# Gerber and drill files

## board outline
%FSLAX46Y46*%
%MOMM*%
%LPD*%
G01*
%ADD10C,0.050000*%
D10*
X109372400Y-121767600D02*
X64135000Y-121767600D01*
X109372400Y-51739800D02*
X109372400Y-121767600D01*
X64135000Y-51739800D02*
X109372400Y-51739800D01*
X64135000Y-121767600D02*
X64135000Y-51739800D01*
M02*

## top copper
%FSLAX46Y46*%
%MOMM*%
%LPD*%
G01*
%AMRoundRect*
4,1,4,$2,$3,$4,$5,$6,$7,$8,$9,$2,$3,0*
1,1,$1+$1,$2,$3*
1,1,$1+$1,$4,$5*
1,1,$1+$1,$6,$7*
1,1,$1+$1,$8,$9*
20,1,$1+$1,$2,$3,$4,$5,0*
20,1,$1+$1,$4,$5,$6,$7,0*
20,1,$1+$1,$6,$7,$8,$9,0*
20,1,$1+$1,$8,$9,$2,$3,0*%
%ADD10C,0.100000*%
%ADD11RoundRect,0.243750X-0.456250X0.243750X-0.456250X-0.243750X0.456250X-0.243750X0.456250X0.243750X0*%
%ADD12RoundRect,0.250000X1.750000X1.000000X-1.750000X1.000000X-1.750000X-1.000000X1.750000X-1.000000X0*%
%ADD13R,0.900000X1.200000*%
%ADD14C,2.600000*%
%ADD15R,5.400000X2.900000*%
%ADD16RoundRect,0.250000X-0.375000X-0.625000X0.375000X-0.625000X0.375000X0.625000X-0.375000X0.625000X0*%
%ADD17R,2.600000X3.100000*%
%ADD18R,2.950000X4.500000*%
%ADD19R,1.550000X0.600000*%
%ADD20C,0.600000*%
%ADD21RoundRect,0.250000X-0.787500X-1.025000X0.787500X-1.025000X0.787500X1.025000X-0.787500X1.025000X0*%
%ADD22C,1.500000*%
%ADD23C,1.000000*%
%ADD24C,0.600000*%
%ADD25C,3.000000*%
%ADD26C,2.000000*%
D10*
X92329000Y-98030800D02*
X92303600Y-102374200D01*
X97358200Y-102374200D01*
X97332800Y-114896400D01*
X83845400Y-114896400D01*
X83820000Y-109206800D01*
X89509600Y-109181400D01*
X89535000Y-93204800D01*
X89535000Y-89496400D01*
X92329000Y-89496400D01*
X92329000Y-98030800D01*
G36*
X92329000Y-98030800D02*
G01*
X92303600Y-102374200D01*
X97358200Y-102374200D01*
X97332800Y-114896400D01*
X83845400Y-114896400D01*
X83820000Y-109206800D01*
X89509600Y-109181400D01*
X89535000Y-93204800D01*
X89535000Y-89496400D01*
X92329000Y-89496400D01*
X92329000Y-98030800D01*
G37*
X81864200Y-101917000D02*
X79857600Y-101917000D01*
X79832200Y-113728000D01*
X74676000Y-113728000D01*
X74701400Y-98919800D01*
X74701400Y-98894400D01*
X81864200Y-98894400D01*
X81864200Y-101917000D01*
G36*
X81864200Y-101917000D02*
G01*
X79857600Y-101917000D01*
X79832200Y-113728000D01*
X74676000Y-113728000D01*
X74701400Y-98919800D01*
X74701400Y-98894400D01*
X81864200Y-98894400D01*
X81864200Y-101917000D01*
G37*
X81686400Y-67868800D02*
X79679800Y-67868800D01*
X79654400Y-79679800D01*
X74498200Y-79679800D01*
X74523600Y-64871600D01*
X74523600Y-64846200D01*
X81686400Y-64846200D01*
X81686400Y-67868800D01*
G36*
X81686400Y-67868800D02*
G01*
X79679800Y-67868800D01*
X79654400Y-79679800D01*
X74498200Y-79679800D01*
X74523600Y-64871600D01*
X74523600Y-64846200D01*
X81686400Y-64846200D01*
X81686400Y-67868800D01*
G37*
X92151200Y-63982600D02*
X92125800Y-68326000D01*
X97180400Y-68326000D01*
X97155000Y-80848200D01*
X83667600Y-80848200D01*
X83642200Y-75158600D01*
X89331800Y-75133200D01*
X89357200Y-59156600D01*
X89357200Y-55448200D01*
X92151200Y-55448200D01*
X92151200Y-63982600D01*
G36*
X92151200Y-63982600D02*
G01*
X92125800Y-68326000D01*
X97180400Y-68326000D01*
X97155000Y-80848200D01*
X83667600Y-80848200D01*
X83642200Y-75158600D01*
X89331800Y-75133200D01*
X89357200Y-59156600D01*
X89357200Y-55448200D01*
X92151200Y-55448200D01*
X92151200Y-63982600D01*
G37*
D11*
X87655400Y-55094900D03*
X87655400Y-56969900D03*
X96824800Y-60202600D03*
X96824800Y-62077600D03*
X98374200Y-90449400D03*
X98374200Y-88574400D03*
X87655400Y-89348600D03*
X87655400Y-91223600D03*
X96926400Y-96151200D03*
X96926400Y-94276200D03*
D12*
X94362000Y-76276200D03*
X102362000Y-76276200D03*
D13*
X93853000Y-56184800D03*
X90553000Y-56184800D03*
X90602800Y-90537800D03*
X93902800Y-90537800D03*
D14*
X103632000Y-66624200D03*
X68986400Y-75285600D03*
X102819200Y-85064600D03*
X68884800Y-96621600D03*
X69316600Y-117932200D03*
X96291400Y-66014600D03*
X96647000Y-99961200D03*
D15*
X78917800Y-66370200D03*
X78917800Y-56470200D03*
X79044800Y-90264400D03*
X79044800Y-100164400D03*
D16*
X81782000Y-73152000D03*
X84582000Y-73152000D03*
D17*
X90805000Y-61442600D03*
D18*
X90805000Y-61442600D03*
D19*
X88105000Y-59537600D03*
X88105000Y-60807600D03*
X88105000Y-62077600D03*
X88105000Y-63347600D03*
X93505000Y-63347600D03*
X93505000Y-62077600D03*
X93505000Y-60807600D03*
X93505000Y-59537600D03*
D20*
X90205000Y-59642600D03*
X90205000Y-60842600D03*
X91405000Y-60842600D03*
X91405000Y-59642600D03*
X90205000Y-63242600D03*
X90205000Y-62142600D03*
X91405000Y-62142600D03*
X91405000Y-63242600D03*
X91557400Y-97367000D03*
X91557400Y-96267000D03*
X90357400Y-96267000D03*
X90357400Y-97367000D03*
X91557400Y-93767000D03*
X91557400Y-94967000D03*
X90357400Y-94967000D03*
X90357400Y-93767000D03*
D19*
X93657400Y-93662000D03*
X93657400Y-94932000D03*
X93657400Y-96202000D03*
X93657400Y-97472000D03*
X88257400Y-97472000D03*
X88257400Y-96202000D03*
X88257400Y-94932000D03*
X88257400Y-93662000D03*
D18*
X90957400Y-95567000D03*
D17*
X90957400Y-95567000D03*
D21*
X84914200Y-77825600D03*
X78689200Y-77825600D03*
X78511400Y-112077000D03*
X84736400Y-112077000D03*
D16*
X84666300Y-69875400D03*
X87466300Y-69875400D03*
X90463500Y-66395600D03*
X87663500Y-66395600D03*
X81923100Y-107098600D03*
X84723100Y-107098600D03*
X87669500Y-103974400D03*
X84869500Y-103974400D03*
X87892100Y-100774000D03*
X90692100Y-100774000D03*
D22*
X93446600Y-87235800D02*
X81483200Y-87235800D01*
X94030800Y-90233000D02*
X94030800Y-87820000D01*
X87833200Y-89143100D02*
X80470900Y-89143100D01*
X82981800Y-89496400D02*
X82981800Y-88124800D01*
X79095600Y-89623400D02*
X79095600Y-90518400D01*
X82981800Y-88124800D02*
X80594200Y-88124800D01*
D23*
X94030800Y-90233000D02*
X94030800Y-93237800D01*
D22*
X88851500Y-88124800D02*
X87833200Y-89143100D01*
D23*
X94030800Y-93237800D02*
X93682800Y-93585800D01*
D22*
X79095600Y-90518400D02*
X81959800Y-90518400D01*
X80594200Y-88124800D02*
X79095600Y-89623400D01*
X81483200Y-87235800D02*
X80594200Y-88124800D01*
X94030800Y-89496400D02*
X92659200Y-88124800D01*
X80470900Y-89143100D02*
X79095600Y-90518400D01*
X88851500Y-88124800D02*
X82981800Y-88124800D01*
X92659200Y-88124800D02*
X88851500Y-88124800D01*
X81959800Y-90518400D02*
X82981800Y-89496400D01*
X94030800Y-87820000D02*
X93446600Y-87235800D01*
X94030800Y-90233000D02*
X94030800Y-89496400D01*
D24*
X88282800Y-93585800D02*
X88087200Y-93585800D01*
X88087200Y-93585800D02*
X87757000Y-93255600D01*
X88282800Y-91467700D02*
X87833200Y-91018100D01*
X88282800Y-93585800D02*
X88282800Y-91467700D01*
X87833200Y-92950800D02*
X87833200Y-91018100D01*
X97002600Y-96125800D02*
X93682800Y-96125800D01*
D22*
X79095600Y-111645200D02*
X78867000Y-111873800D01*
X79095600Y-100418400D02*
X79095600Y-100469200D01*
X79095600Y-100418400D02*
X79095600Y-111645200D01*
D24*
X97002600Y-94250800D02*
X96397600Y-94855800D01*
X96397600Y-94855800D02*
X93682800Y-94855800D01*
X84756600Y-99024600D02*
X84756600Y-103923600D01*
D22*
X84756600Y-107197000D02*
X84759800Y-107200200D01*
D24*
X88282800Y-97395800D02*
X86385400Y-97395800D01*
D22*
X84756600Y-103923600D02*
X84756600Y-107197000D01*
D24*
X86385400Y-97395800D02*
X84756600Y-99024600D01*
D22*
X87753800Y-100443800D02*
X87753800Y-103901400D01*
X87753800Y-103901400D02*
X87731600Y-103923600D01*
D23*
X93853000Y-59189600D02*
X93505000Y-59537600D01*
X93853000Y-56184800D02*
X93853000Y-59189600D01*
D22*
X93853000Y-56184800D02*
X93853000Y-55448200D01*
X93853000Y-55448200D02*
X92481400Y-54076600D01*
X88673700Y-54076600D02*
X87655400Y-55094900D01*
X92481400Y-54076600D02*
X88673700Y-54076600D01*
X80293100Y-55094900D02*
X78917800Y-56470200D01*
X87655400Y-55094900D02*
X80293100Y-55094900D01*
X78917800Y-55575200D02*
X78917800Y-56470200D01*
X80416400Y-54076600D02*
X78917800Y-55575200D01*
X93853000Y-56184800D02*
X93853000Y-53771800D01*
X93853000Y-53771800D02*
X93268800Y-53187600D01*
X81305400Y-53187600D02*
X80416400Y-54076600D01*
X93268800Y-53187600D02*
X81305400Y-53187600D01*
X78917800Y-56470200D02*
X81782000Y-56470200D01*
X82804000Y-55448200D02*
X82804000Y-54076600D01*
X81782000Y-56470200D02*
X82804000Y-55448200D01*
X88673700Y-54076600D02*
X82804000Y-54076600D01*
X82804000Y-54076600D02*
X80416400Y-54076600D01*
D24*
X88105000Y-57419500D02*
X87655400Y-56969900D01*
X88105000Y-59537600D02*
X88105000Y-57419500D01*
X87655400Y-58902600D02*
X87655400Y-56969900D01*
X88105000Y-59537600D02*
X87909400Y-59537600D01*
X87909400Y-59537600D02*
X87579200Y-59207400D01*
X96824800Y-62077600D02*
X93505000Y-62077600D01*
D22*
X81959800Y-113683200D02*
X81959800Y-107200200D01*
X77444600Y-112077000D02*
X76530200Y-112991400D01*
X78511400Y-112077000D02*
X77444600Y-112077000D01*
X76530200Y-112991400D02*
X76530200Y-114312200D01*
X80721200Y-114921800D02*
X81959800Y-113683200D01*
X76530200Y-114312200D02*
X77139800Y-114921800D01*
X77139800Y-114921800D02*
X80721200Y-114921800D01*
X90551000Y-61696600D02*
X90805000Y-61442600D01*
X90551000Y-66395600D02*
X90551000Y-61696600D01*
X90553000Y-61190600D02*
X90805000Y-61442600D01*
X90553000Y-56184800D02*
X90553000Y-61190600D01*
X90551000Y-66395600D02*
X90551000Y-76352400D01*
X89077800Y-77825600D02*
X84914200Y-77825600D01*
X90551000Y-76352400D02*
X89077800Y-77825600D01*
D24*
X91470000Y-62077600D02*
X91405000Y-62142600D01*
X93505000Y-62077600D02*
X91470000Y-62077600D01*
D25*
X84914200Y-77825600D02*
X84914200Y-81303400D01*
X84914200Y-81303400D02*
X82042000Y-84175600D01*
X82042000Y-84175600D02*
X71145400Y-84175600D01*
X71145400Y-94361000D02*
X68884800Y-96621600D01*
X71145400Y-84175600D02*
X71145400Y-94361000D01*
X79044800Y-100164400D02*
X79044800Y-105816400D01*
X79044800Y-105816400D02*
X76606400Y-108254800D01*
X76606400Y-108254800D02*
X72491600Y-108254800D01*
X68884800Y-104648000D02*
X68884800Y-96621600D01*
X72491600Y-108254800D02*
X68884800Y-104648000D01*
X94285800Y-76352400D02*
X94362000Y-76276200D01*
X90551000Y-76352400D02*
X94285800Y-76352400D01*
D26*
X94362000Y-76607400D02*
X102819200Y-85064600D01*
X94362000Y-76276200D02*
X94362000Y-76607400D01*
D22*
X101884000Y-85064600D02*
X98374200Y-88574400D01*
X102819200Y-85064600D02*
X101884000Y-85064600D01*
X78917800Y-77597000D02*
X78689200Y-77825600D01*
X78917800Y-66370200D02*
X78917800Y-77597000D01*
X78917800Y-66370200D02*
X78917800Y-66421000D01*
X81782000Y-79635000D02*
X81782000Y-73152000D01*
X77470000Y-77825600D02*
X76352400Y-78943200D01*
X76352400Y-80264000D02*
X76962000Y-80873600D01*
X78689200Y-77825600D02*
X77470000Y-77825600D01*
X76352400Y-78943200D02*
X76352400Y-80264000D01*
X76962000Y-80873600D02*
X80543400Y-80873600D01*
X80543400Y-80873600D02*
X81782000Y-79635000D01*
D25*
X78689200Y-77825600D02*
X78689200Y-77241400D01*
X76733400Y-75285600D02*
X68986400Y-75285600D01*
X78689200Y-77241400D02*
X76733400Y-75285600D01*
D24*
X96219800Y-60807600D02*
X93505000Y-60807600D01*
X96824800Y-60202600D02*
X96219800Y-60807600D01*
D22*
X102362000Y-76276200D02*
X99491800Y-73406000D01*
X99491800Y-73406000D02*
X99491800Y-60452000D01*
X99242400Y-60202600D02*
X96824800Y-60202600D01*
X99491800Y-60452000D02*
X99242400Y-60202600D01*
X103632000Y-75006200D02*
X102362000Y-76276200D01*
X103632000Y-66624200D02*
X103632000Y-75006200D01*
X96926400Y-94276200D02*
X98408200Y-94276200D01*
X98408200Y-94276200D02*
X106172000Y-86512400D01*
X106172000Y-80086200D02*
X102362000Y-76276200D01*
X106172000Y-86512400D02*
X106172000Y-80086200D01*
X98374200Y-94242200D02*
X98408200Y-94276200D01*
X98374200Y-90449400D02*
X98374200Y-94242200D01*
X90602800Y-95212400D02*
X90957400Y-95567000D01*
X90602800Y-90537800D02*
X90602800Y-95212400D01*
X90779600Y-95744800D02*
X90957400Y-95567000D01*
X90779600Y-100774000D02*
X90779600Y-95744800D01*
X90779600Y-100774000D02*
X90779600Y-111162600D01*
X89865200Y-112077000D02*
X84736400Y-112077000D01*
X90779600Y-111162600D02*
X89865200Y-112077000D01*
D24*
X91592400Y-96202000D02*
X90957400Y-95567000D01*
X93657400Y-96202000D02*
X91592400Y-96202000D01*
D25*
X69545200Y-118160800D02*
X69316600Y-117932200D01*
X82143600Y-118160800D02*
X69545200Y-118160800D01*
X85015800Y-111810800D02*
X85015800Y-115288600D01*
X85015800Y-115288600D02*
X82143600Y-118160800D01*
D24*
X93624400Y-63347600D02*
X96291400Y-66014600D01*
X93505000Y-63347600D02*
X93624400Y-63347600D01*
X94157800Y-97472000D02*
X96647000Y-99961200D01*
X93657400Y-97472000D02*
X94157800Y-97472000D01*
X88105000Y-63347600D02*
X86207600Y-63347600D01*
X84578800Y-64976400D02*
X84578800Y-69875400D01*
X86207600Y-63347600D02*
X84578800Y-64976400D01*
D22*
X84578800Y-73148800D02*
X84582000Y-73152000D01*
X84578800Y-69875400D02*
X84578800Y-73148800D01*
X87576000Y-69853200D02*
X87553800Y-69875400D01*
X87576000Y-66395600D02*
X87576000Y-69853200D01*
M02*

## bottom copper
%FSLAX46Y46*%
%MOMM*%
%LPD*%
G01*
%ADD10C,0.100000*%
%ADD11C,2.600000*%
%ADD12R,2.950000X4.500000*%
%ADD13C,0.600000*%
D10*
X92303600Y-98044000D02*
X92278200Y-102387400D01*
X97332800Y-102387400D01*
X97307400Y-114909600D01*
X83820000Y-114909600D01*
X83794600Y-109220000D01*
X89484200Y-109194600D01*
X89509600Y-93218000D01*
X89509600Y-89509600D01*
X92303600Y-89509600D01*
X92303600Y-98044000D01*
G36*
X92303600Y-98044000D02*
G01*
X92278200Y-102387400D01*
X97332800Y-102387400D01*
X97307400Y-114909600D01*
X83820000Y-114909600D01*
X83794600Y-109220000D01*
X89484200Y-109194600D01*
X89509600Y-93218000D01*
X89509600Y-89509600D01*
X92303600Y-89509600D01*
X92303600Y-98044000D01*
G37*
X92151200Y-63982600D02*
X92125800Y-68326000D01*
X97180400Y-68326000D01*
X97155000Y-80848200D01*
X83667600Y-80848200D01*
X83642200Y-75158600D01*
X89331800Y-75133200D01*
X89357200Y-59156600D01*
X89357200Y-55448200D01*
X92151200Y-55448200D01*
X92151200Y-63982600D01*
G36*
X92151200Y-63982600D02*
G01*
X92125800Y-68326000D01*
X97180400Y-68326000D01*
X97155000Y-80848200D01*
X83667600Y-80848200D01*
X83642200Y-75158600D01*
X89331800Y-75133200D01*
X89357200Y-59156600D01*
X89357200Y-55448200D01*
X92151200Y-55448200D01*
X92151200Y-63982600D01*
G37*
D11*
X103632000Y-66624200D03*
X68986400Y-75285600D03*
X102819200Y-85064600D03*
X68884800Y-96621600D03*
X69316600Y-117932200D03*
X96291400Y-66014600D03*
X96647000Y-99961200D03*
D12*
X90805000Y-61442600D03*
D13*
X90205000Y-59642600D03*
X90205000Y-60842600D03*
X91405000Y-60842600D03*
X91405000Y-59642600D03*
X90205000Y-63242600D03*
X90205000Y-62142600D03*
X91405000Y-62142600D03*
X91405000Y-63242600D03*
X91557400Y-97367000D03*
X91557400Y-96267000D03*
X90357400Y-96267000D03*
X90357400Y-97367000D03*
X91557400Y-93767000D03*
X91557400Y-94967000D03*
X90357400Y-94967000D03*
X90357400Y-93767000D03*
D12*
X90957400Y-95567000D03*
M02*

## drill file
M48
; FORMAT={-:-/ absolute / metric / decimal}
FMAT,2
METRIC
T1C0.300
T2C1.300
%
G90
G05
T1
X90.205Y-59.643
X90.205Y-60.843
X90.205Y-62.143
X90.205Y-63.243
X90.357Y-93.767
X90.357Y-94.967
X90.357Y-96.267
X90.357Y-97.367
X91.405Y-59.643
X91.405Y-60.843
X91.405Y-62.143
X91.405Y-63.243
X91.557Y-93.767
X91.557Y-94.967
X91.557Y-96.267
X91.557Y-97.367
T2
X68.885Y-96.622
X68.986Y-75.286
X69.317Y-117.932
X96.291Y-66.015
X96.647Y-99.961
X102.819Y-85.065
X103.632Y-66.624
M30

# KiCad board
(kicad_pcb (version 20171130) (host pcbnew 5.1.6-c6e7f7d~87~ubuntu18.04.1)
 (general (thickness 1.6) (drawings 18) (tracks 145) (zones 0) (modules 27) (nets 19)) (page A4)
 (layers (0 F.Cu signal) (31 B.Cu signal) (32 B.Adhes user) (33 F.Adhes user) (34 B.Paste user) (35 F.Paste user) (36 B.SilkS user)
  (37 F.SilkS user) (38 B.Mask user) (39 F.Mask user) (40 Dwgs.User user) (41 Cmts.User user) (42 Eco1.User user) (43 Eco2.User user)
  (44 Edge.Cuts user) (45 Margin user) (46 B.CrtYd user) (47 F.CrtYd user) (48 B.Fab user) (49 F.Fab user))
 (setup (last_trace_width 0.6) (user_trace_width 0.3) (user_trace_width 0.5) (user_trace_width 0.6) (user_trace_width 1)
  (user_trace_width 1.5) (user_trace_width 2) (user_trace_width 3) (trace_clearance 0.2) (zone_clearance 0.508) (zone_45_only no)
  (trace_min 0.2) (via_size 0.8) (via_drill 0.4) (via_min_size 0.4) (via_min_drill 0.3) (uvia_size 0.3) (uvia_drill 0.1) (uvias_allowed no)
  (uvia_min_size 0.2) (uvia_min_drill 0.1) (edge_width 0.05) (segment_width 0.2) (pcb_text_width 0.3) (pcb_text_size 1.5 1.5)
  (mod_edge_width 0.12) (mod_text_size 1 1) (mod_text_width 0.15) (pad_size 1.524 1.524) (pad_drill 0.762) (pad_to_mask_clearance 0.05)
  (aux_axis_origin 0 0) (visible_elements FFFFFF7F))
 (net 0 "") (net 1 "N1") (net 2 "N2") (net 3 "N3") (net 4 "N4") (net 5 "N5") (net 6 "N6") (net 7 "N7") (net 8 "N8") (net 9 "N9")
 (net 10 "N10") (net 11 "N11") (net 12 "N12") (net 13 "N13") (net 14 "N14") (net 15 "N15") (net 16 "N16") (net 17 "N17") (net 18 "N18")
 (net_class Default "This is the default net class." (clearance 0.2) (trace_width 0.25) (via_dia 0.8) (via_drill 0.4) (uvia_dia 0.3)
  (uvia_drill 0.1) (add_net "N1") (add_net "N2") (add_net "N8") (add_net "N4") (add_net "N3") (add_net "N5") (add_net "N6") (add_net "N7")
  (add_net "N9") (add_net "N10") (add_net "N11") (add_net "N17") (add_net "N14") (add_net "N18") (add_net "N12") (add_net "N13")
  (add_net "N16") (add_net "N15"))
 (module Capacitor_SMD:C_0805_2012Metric (layer F.Cu) (at 87.6554 56.0324 270)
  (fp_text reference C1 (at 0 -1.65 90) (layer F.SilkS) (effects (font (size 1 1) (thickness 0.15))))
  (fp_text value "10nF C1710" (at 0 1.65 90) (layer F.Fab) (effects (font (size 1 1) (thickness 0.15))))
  (pad 1 smd roundrect (at -0.9375 0 270) (size 0.975 1.4) (layers F.Cu F.Paste F.Mask) (roundrect_rratio 0.25) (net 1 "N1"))
  (pad 2 smd roundrect (at 0.9375 0 270) (size 0.975 1.4) (layers F.Cu F.Paste F.Mask) (roundrect_rratio 0.25) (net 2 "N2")))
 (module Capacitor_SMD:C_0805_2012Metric (layer F.Cu) (at 96.8248 61.1401 270)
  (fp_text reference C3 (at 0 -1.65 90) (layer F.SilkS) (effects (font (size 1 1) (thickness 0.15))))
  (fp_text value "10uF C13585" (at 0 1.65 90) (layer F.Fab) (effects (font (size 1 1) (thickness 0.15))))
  (pad 1 smd roundrect (at -0.9375 0 270) (size 0.975 1.4) (layers F.Cu F.Paste F.Mask) (roundrect_rratio 0.25) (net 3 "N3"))
  (pad 2 smd roundrect (at 0.9375 0 270) (size 0.975 1.4) (layers F.Cu F.Paste F.Mask) (roundrect_rratio 0.25) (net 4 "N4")))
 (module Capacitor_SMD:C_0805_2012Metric (layer F.Cu) (at 98.3742 89.5119 270)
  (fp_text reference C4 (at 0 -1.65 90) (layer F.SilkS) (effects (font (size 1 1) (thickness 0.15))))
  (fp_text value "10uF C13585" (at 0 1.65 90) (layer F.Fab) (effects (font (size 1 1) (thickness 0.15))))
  (pad 2 smd roundrect (at 0.9375 0 270) (size 0.975 1.4) (layers F.Cu F.Paste F.Mask) (roundrect_rratio 0.25) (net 3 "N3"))
  (pad 1 smd roundrect (at -0.9375 0 270) (size 0.975 1.4) (layers F.Cu F.Paste F.Mask) (roundrect_rratio 0.25) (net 4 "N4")))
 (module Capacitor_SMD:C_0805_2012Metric (layer F.Cu) (at 87.6554 90.2861 270)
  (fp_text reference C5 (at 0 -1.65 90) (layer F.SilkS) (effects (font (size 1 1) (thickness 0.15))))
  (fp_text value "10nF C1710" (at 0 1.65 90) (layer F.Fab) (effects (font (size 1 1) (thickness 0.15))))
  (pad 1 smd roundrect (at -0.9375 0 270) (size 0.975 1.4) (layers F.Cu F.Paste F.Mask) (roundrect_rratio 0.25) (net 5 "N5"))
  (pad 2 smd roundrect (at 0.9375 0 270) (size 0.975 1.4) (layers F.Cu F.Paste F.Mask) (roundrect_rratio 0.25) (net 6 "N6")))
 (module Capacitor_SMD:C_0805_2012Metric (layer F.Cu) (at 96.9264 95.2137 270)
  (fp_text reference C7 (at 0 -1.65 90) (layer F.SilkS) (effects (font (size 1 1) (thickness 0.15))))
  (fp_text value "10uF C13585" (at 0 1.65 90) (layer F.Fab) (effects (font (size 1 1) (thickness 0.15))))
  (pad 2 smd roundrect (at 0.9375 0 270) (size 0.975 1.4) (layers F.Cu F.Paste F.Mask) (roundrect_rratio 0.25) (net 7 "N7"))
  (pad 1 smd roundrect (at -0.9375 0 270) (size 0.975 1.4) (layers F.Cu F.Paste F.Mask) (roundrect_rratio 0.25) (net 3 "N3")))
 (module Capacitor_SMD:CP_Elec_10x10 (layer F.Cu) (at 98.362 76.2762 180)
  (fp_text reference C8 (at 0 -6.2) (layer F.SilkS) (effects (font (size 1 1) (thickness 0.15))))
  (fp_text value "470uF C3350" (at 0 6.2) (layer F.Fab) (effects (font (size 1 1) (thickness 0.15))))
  (pad 2 smd roundrect (at 4 0 180) (size 4 2.5) (layers F.Cu F.Paste F.Mask) (roundrect_rratio 0.1) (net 4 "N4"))
  (pad 1 smd roundrect (at -4 0 180) (size 4 2.5) (layers F.Cu F.Paste F.Mask) (roundrect_rratio 0.1) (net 3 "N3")))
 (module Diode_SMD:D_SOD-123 (layer F.Cu) (at 92.203 56.1848 180)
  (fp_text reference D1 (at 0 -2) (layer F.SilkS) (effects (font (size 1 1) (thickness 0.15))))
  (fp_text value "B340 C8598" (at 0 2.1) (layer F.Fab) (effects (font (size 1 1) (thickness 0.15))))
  (pad 1 smd rect (at -1.65 0 180) (size 0.9 1.2) (layers F.Cu F.Paste F.Mask) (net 1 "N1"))
  (pad 2 smd rect (at 1.65 0 180) (size 0.9 1.2) (layers F.Cu F.Paste F.Mask) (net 4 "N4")))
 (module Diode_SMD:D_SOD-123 (layer F.Cu) (at 92.2528 90.5378 180)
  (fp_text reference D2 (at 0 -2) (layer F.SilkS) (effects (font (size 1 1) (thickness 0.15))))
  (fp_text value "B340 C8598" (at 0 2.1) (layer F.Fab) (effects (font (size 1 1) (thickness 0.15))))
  (pad 2 smd rect (at 1.65 0 180) (size 0.9 1.2) (layers F.Cu F.Paste F.Mask) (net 7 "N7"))
  (pad 1 smd rect (at -1.65 0 180) (size 0.9 1.2) (layers F.Cu F.Paste F.Mask) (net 5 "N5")))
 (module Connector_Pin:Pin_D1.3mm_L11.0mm (layer F.Cu) (at 103.632 66.6242)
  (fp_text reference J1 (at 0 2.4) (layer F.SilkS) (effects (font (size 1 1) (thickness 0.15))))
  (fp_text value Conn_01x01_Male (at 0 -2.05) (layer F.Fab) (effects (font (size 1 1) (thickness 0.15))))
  (pad 1 thru_hole circle (at 0 0) (size 2.6 2.6) (drill 1.3) (layers *.Cu *.Mask) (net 3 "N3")))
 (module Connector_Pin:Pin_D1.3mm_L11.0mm (layer F.Cu) (at 68.9864 75.2856)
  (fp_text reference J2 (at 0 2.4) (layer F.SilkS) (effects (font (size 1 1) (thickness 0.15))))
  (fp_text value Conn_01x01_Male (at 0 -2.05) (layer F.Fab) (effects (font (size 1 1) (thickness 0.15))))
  (pad 1 thru_hole circle (at 0 0) (size 2.6 2.6) (drill 1.3) (layers *.Cu *.Mask) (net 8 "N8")))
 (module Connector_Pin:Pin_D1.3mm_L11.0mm (layer F.Cu) (at 102.8192 85.0646)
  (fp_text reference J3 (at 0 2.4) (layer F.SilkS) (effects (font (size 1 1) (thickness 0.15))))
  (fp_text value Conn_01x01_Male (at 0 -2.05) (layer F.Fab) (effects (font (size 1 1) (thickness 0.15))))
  (pad 1 thru_hole circle (at 0 0) (size 2.6 2.6) (drill 1.3) (layers *.Cu *.Mask) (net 4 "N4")))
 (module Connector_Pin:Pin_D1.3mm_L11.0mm (layer F.Cu) (at 68.8848 96.6216)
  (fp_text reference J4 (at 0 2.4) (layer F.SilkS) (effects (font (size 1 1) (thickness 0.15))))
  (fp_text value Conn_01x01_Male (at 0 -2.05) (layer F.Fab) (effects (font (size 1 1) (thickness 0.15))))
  (pad 1 thru_hole circle (at 0 0) (size 2.6 2.6) (drill 1.3) (layers *.Cu *.Mask) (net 4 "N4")))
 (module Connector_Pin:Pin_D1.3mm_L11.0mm (layer F.Cu) (at 69.3166 117.9322)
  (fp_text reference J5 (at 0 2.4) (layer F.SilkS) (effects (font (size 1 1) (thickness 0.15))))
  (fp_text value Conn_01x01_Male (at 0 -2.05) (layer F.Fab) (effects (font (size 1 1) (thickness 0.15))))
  (pad 1 thru_hole circle (at 0 0) (size 2.6 2.6) (drill 1.3) (layers *.Cu *.Mask) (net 7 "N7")))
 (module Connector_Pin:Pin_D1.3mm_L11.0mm (layer F.Cu) (at 96.2914 66.0146)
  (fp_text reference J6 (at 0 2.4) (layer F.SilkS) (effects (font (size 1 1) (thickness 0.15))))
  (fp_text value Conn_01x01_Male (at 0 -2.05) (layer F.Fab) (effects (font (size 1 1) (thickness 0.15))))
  (pad 1 thru_hole circle (at 0 0) (size 2.6 2.6) (drill 1.3) (layers *.Cu *.Mask) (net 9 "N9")))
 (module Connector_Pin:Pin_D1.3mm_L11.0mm (layer F.Cu) (at 96.647 99.9612)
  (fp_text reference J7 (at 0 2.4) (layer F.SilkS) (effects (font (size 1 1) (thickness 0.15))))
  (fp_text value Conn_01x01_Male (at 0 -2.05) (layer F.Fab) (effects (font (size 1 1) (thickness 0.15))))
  (pad 1 thru_hole circle (at 0 0) (size 2.6 2.6) (drill 1.3) (layers *.Cu *.Mask) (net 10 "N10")))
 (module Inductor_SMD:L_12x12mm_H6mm (layer F.Cu) (at 78.9178 61.4202 90)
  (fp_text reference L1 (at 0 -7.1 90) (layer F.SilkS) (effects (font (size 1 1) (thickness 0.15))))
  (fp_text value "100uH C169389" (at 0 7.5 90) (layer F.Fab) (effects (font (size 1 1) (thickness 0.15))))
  (pad 1 smd rect (at -4.95 0 90) (size 2.9 5.4) (layers F.Cu F.Paste F.Mask) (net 8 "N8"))
  (pad 2 smd rect (at 4.95 0 90) (size 2.9 5.4) (layers F.Cu F.Paste F.Mask) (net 1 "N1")))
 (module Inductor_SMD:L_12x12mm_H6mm (layer F.Cu) (at 79.0448 95.2144 90)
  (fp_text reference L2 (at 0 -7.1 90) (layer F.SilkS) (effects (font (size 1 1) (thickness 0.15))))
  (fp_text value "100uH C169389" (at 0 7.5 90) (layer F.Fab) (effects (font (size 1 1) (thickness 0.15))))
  (pad 2 smd rect (at 4.95 0 90) (size 2.9 5.4) (layers F.Cu F.Paste F.Mask) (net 5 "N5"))
  (pad 1 smd rect (at -4.95 0 90) (size 2.9 5.4) (layers F.Cu F.Paste F.Mask) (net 4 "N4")))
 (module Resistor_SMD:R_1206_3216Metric (layer F.Cu) (at 83.182 73.152)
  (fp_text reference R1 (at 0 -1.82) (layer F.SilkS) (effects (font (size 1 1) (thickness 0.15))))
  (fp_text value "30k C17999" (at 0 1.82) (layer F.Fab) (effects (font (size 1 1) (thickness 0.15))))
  (pad 1 smd roundrect (at -1.4 0) (size 1.25 1.75) (layers F.Cu F.Paste F.Mask) (roundrect_rratio 0.2) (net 8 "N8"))
  (pad 2 smd roundrect (at 1.4 0) (size 1.25 1.75) (layers F.Cu F.Paste F.Mask) (roundrect_rratio 0.2) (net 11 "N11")))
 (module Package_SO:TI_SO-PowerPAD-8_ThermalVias (layer F.Cu) (at 90.805 61.4426)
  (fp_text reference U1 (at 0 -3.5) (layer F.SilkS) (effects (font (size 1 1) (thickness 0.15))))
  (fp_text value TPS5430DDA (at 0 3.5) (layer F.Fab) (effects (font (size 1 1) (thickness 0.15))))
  (pad 9 smd rect (at 0 0) (size 2.6 3.1) (layers F.Cu F.Paste F.Mask) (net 4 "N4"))
  (pad 9 smd rect (at 0 0) (size 2.95 4.5) (layers F.Cu) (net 4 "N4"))
  (pad 1 smd rect (at -2.7 -1.905) (size 1.55 0.6) (layers F.Cu F.Paste F.Mask) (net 2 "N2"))
  (pad 2 smd rect (at -2.7 -0.635) (size 1.55 0.6) (layers F.Cu F.Paste F.Mask) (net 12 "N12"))
  (pad 3 smd rect (at -2.7 0.635) (size 1.55 0.6) (layers F.Cu F.Paste F.Mask) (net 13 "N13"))
  (pad 4 smd rect (at -2.7 1.905) (size 1.55 0.6) (layers F.Cu F.Paste F.Mask) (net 11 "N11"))
  (pad 5 smd rect (at 2.7 1.905) (size 1.55 0.6) (layers F.Cu F.Paste F.Mask) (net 9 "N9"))
  (pad 6 smd rect (at 2.7 0.635) (size 1.55 0.6) (layers F.Cu F.Paste F.Mask) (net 4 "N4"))
  (pad 7 smd rect (at 2.7 -0.635) (size 1.55 0.6) (layers F.Cu F.Paste F.Mask) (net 3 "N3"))
  (pad 8 smd rect (at 2.7 -1.905) (size 1.55 0.6) (layers F.Cu F.Paste F.Mask) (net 1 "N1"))
  (pad 9 smd rect (at 0 0) (size 2.95 4.5) (layers B.Cu) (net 4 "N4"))
  (pad 9 thru_hole circle (at -0.6 -1.8) (size 0.6 0.6) (drill 0.3) (layers *.Cu) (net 4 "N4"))
  (pad 9 thru_hole circle (at -0.6 -0.6) (size 0.6 0.6) (drill 0.3) (layers *.Cu) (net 4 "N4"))
  (pad 9 thru_hole circle (at 0.6 -0.6) (size 0.6 0.6) (drill 0.3) (layers *.Cu) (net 4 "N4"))
  (pad 9 thru_hole circle (at 0.6 -1.8) (size 0.6 0.6) (drill 0.3) (layers *.Cu) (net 4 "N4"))
  (pad 9 thru_hole circle (at -0.6 1.8) (size 0.6 0.6) (drill 0.3) (layers *.Cu) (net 4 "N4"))
  (pad 9 thru_hole circle (at -0.6 0.7) (size 0.6 0.6) (drill 0.3) (layers *.Cu) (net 4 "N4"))
  (pad 9 thru_hole circle (at 0.6 0.7) (size 0.6 0.6) (drill 0.3) (layers *.Cu) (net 4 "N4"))
  (pad 9 thru_hole circle (at 0.6 1.8) (size 0.6 0.6) (drill 0.3) (layers *.Cu) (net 4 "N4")))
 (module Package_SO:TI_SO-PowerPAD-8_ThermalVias (layer F.Cu) (at 90.9574 95.567)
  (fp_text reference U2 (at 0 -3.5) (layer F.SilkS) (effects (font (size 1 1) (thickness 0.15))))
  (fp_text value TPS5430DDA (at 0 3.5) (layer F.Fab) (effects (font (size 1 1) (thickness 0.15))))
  (pad 9 thru_hole circle (at 0.6 1.8) (size 0.6 0.6) (drill 0.3) (layers *.Cu) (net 7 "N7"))
  (pad 9 thru_hole circle (at 0.6 0.7) (size 0.6 0.6) (drill 0.3) (layers *.Cu) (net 7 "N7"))
  (pad 9 thru_hole circle (at -0.6 0.7) (size 0.6 0.6) (drill 0.3) (layers *.Cu) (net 7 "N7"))
  (pad 9 thru_hole circle (at -0.6 1.8) (size 0.6 0.6) (drill 0.3) (layers *.Cu) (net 7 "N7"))
  (pad 9 thru_hole circle (at 0.6 -1.8) (size 0.6 0.6) (drill 0.3) (layers *.Cu) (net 7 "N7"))
  (pad 9 thru_hole circle (at 0.6 -0.6) (size 0.6 0.6) (drill 0.3) (layers *.Cu) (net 7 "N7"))
  (pad 9 thru_hole circle (at -0.6 -0.6) (size 0.6 0.6) (drill 0.3) (layers *.Cu) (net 7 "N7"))
  (pad 9 thru_hole circle (at -0.6 -1.8) (size 0.6 0.6) (drill 0.3) (layers *.Cu) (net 7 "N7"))
  (pad 9 smd rect (at 0 0) (size 2.95 4.5) (layers B.Cu) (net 7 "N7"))
  (pad 8 smd rect (at 2.7 -1.905) (size 1.55 0.6) (layers F.Cu F.Paste F.Mask) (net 5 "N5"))
  (pad 7 smd rect (at 2.7 -0.635) (size 1.55 0.6) (layers F.Cu F.Paste F.Mask) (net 3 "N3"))
  (pad 6 smd rect (at 2.7 0.635) (size 1.55 0.6) (layers F.Cu F.Paste F.Mask) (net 7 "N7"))
  (pad 5 smd rect (at 2.7 1.905) (size 1.55 0.6) (layers F.Cu F.Paste F.Mask) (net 10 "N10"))
  (pad 4 smd rect (at -2.7 1.905) (size 1.55 0.6) (layers F.Cu F.Paste F.Mask) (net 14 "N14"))
  (pad 3 smd rect (at -2.7 0.635) (size 1.55 0.6) (layers F.Cu F.Paste F.Mask) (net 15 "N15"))
  (pad 2 smd rect (at -2.7 -0.635) (size 1.55 0.6) (layers F.Cu F.Paste F.Mask) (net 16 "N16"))
  (pad 1 smd rect (at -2.7 -1.905) (size 1.55 0.6) (layers F.Cu F.Paste F.Mask) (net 6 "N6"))
  (pad 9 smd rect (at 0 0) (size 2.95 4.5) (layers F.Cu) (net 7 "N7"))
  (pad 9 smd rect (at 0 0) (size 2.6 3.1) (layers F.Cu F.Paste F.Mask) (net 7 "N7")))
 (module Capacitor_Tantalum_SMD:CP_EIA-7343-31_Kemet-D (layer F.Cu) (at 81.8017 77.8256)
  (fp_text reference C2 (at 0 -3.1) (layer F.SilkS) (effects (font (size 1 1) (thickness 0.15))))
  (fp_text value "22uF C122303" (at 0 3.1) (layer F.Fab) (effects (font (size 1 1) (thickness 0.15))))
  (pad 2 smd roundrect (at 3.1125 0) (size 2.075 2.55) (layers F.Cu F.Paste F.Mask) (roundrect_rratio 0.120482) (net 4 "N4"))
  (pad 1 smd roundrect (at -3.1125 0) (size 2.075 2.55) (layers F.Cu F.Paste F.Mask) (roundrect_rratio 0.120482) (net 8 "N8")))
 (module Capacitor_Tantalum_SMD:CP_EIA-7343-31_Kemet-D (layer F.Cu) (at 81.6239 112.077)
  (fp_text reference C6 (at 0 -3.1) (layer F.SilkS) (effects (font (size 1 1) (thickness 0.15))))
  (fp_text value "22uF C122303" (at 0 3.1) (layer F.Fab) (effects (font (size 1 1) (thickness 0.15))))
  (pad 1 smd roundrect (at -3.1125 0) (size 2.075 2.55) (layers F.Cu F.Paste F.Mask) (roundrect_rratio 0.120482) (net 4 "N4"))
  (pad 2 smd roundrect (at 3.1125 0) (size 2.075 2.55) (layers F.Cu F.Paste F.Mask) (roundrect_rratio 0.120482) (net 7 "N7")))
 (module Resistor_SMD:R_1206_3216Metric (layer F.Cu) (at 86.0663 69.8754)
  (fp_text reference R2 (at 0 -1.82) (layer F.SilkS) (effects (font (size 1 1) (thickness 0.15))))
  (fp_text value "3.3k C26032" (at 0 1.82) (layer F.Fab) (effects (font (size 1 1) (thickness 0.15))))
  (pad 1 smd roundrect (at -1.4 0) (size 1.25 1.75) (layers F.Cu F.Paste F.Mask) (roundrect_rratio 0.2) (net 11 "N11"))
  (pad 2 smd roundrect (at 1.4 0) (size 1.25 1.75) (layers F.Cu F.Paste F.Mask) (roundrect_rratio 0.2) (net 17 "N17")))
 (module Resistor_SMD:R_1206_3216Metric (layer F.Cu) (at 89.0635 66.3956)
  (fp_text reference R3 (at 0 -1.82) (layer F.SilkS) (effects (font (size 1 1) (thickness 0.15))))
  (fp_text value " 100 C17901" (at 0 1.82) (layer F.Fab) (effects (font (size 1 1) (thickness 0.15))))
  (pad 2 smd roundrect (at 1.4 0) (size 1.25 1.75) (layers F.Cu F.Paste F.Mask) (roundrect_rratio 0.2) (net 4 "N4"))
  (pad 1 smd roundrect (at -1.4 0) (size 1.25 1.75) (layers F.Cu F.Paste F.Mask) (roundrect_rratio 0.2) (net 17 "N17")))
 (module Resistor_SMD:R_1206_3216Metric (layer F.Cu) (at 83.3231 107.0986)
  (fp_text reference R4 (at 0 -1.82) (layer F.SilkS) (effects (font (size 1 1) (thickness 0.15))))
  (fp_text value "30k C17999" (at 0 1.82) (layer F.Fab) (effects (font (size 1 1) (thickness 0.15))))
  (pad 1 smd roundrect (at -1.4 0) (size 1.25 1.75) (layers F.Cu F.Paste F.Mask) (roundrect_rratio 0.2) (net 4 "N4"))
  (pad 2 smd roundrect (at 1.4 0) (size 1.25 1.75) (layers F.Cu F.Paste F.Mask) (roundrect_rratio 0.2) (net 14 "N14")))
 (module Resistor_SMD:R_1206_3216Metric (layer F.Cu) (at 86.2695 103.9744)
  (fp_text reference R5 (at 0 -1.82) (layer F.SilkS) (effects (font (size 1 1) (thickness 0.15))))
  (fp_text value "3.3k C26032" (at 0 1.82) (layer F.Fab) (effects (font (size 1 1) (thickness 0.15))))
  (pad 2 smd roundrect (at 1.4 0) (size 1.25 1.75) (layers F.Cu F.Paste F.Mask) (roundrect_rratio 0.2) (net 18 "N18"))
  (pad 1 smd roundrect (at -1.4 0) (size 1.25 1.75) (layers F.Cu F.Paste F.Mask) (roundrect_rratio 0.2) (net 14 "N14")))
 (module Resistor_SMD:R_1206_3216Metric (layer F.Cu) (at 89.2921 100.774)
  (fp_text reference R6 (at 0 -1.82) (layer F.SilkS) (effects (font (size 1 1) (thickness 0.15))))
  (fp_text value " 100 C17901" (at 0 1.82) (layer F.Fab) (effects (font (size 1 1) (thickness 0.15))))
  (pad 1 smd roundrect (at -1.4 0) (size 1.25 1.75) (layers F.Cu F.Paste F.Mask) (roundrect_rratio 0.2) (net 18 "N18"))
  (pad 2 smd roundrect (at 1.4 0) (size 1.25 1.75) (layers F.Cu F.Paste F.Mask) (roundrect_rratio 0.2) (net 7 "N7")))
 (gr_poly
  (pts (xy 92.3036 98.044) (xy 92.2782 102.3874) (xy 97.3328 102.3874) (xy 97.3074 114.9096) (xy 83.82 114.9096) (xy 83.7946 109.22)
   (xy 89.4842 109.1946) (xy 89.5096 93.218) (xy 89.5096 89.5096) (xy 92.3036 89.5096))
  (layer B.Cu) (width 0.1))
 (gr_poly
  (pts (xy 92.1512 63.9826) (xy 92.1258 68.326) (xy 97.1804 68.326) (xy 97.155 80.8482) (xy 83.6676 80.8482) (xy 83.6422 75.1586)
   (xy 89.3318 75.1332) (xy 89.3572 59.1566) (xy 89.3572 55.4482) (xy 92.1512 55.4482))
  (layer B.Cu) (width 0.1))
 (gr_line (start 109.3724 121.7676) (end 64.135 121.7676) (layer Edge.Cuts) (width 0.05))
 (gr_line (start 109.3724 51.7398) (end 109.3724 121.7676) (layer Edge.Cuts) (width 0.05))
 (gr_line (start 64.135 51.7398) (end 109.3724 51.7398) (layer Edge.Cuts) (width 0.05))
 (gr_line (start 64.135 121.7676) (end 64.135 51.7398) (layer Edge.Cuts) (width 0.05))
 (gr_poly
  (pts (xy 92.329 98.0308) (xy 92.3036 102.3742) (xy 97.3582 102.3742) (xy 97.3328 114.8964) (xy 83.8454 114.8964) (xy 83.82 109.2068)
   (xy 89.5096 109.1814) (xy 89.535 93.2048) (xy 89.535 89.4964) (xy 92.329 89.4964))
  (layer F.Cu) (width 0.1))
 (gr_poly
  (pts (xy 81.8642 101.917) (xy 79.8576 101.917) (xy 79.8322 113.728) (xy 74.676 113.728) (xy 74.7014 98.9198) (xy 74.7014 98.8944)
   (xy 81.8642 98.8944))
  (layer F.Cu) (width 0.1))
 (gr_poly
  (pts (xy 81.6864 67.8688) (xy 79.6798 67.8688) (xy 79.6544 79.6798) (xy 74.4982 79.6798) (xy 74.5236 64.8716) (xy 74.5236 64.8462)
   (xy 81.6864 64.8462))
  (layer F.Cu) (width 0.1))
 (gr_poly
  (pts (xy 92.1512 63.9826) (xy 92.1258 68.326) (xy 97.1804 68.326) (xy 97.155 80.8482) (xy 83.6676 80.8482) (xy 83.6422 75.1586)
   (xy 89.3318 75.1332) (xy 89.3572 59.1566) (xy 89.3572 55.4482) (xy 92.1512 55.4482))
  (layer F.Cu) (width 0.1))
 (segment (start 93.4466 87.2358) (end 81.4832 87.2358) (width 1.5) (layer F.Cu) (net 5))
 (segment (start 94.0308 90.233) (end 94.0308 87.82) (width 1.5) (layer F.Cu) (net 5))
 (segment (start 87.8332 89.1431) (end 80.4709 89.1431) (width 1.5) (layer F.Cu) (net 5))
 (segment (start 82.9818 89.4964) (end 82.9818 88.1248) (width 1.5) (layer F.Cu) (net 5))
 (segment (start 79.0956 89.6234) (end 79.0956 90.5184) (width 1.5) (layer F.Cu) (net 5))
 (segment (start 82.9818 88.1248) (end 80.5942 88.1248) (width 1.5) (layer F.Cu) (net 5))
 (segment (start 94.0308 90.233) (end 94.0308 93.2378) (width 1) (layer F.Cu) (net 5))
 (segment (start 88.8515 88.1248) (end 87.8332 89.1431) (width 1.5) (layer F.Cu) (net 5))
 (segment (start 94.0308 93.2378) (end 93.6828 93.5858) (width 1) (layer F.Cu) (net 5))
 (segment (start 79.0956 90.5184) (end 81.9598 90.5184) (width 1.5) (layer F.Cu) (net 5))
 (segment (start 80.5942 88.1248) (end 79.0956 89.6234) (width 1.5) (layer F.Cu) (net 5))
 (segment (start 81.4832 87.2358) (end 80.5942 88.1248) (width 1.5) (layer F.Cu) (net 5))
 (segment (start 94.0308 89.4964) (end 92.6592 88.1248) (width 1.5) (layer F.Cu) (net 5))
 (segment (start 80.4709 89.1431) (end 79.0956 90.5184) (width 1.5) (layer F.Cu) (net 5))
 (segment (start 88.8515 88.1248) (end 82.9818 88.1248) (width 1.5) (layer F.Cu) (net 5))
 (segment (start 92.6592 88.1248) (end 88.8515 88.1248) (width 1.5) (layer F.Cu) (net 5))
 (segment (start 81.9598 90.5184) (end 82.9818 89.4964) (width 1.5) (layer F.Cu) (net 5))
 (segment (start 94.0308 87.82) (end 93.4466 87.2358) (width 1.5) (layer F.Cu) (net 5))
 (segment (start 94.0308 90.233) (end 94.0308 89.4964) (width 1.5) (layer F.Cu) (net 5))
 (segment (start 88.2828 93.5858) (end 88.0872 93.5858) (width 0.6) (layer F.Cu) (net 6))
 (segment (start 88.0872 93.5858) (end 87.757 93.2556) (width 0.6) (layer F.Cu) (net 6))
 (segment (start 88.2828 91.4677) (end 87.8332 91.0181) (width 0.6) (layer F.Cu) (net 6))
 (segment (start 88.2828 93.5858) (end 88.2828 91.4677) (width 0.6) (layer F.Cu) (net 6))
 (segment (start 87.8332 92.9508) (end 87.8332 91.0181) (width 0.6) (layer F.Cu) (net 6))
 (segment (start 97.0026 96.1258) (end 93.6828 96.1258) (width 0.6) (layer F.Cu) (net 7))
 (segment (start 79.0956 111.6452) (end 78.867 111.8738) (width 1.5) (layer F.Cu) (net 4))
 (segment (start 79.0956 100.4184) (end 79.0956 100.4692) (width 1.5) (layer F.Cu) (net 4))
 (segment (start 79.0956 100.4184) (end 79.0956 111.6452) (width 1.5) (layer F.Cu) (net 4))
 (segment (start 97.0026 94.2508) (end 96.3976 94.8558) (width 0.6) (layer F.Cu) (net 3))
 (segment (start 96.3976 94.8558) (end 93.6828 94.8558) (width 0.6) (layer F.Cu) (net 3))
 (segment (start 84.7566 99.0246) (end 84.7566 103.9236) (width 0.6) (layer F.Cu) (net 14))
 (segment (start 84.7566 107.197) (end 84.7598 107.2002) (width 1.5) (layer F.Cu) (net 14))
 (segment (start 88.2828 97.3958) (end 86.3854 97.3958) (width 0.6) (layer F.Cu) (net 14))
 (segment (start 84.7566 103.9236) (end 84.7566 107.197) (width 1.5) (layer F.Cu) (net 14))
 (segment (start 86.3854 97.3958) (end 84.7566 99.0246) (width 0.6) (layer F.Cu) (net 14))
 (segment (start 87.7538 100.4438) (end 87.7538 103.9014) (width 1.5) (layer F.Cu) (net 18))
 (segment (start 87.7538 103.9014) (end 87.7316 103.9236) (width 1.5) (layer F.Cu) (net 18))
 (segment (start 93.853 59.1896) (end 93.505 59.5376) (width 1) (layer F.Cu) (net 1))
 (segment (start 93.853 56.1848) (end 93.853 59.1896) (width 1) (layer F.Cu) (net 1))
 (segment (start 93.853 56.1848) (end 93.853 55.4482) (width 1.5) (layer F.Cu) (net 1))
 (segment (start 93.853 55.4482) (end 92.4814 54.0766) (width 1.5) (layer F.Cu) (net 1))
 (segment (start 88.6737 54.0766) (end 87.6554 55.0949) (width 1.5) (layer F.Cu) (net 1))
 (segment (start 92.4814 54.0766) (end 88.6737 54.0766) (width 1.5) (layer F.Cu) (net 1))
 (segment (start 80.2931 55.0949) (end 78.9178 56.4702) (width 1.5) (layer F.Cu) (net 1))
 (segment (start 87.6554 55.0949) (end 80.2931 55.0949) (width 1.5) (layer F.Cu) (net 1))
 (segment (start 78.9178 55.5752) (end 78.9178 56.4702) (width 1.5) (layer F.Cu) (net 1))
 (segment (start 80.4164 54.0766) (end 78.9178 55.5752) (width 1.5) (layer F.Cu) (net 1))
 (segment (start 93.853 56.1848) (end 93.853 53.7718) (width 1.5) (layer F.Cu) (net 1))
 (segment (start 93.853 53.7718) (end 93.2688 53.1876) (width 1.5) (layer F.Cu) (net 1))
 (segment (start 81.3054 53.1876) (end 80.4164 54.0766) (width 1.5) (layer F.Cu) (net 1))
 (segment (start 93.2688 53.1876) (end 81.3054 53.1876) (width 1.5) (layer F.Cu) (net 1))
 (segment (start 78.9178 56.4702) (end 81.782 56.4702) (width 1.5) (layer F.Cu) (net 1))
 (segment (start 82.804 55.4482) (end 82.804 54.0766) (width 1.5) (layer F.Cu) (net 1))
 (segment (start 81.782 56.4702) (end 82.804 55.4482) (width 1.5) (layer F.Cu) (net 1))
 (segment (start 88.6737 54.0766) (end 82.804 54.0766) (width 1.5) (layer F.Cu) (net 1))
 (segment (start 82.804 54.0766) (end 80.4164 54.0766) (width 1.5) (layer F.Cu) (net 1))
 (segment (start 88.105 57.4195) (end 87.6554 56.9699) (width 0.6) (layer F.Cu) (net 2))
 (segment (start 88.105 59.5376) (end 88.105 57.4195) (width 0.6) (layer F.Cu) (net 2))
 (segment (start 87.6554 58.9026) (end 87.6554 56.9699) (width 0.6) (layer F.Cu) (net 2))
 (segment (start 88.105 59.5376) (end 87.9094 59.5376) (width 0.6) (layer F.Cu) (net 2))
 (segment (start 87.9094 59.5376) (end 87.5792 59.2074) (width 0.6) (layer F.Cu) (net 2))
 (segment (start 96.8248 62.0776) (end 93.505 62.0776) (width 0.6) (layer F.Cu) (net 4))
 (segment (start 81.9598 113.6832) (end 81.9598 107.2002) (width 1.5) (layer F.Cu) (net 4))
 (segment (start 77.4446 112.077) (end 76.5302 112.9914) (width 1.5) (layer F.Cu) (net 4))
 (segment (start 78.5114 112.077) (end 77.4446 112.077) (width 1.5) (layer F.Cu) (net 4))
 (segment (start 76.5302 112.9914) (end 76.5302 114.3122) (width 1.5) (layer F.Cu) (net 4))
 (segment (start 80.7212 114.9218) (end 81.9598 113.6832) (width 1.5) (layer F.Cu) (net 4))
 (segment (start 76.5302 114.3122) (end 77.1398 114.9218) (width 1.5) (layer F.Cu) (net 4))
 (segment (start 77.1398 114.9218) (end 80.7212 114.9218) (width 1.5) (layer F.Cu) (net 4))
 (segment (start 90.551 61.6966) (end 90.805 61.4426) (width 1.5) (layer F.Cu) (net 4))
 (segment (start 90.551 66.3956) (end 90.551 61.6966) (width 1.5) (layer F.Cu) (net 4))
 (segment (start 90.553 61.1906) (end 90.805 61.4426) (width 1.5) (layer F.Cu) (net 4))
 (segment (start 90.553 56.1848) (end 90.553 61.1906) (width 1.5) (layer F.Cu) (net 4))
 (segment (start 90.551 66.3956) (end 90.551 76.3524) (width 1.5) (layer F.Cu) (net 4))
 (segment (start 89.0778 77.8256) (end 84.9142 77.8256) (width 1.5) (layer F.Cu) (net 4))
 (segment (start 90.551 76.3524) (end 89.0778 77.8256) (width 1.5) (layer F.Cu) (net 4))
 (segment (start 91.47 62.0776) (end 91.405 62.1426) (width 0.6) (layer F.Cu) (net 4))
 (segment (start 93.505 62.0776) (end 91.47 62.0776) (width 0.6) (layer F.Cu) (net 4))
 (segment (start 84.9142 77.8256) (end 84.9142 81.3034) (width 3) (layer F.Cu) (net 4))
 (segment (start 84.9142 81.3034) (end 82.042 84.1756) (width 3) (layer F.Cu) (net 4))
 (segment (start 82.042 84.1756) (end 71.1454 84.1756) (width 3) (layer F.Cu) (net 4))
 (segment (start 71.1454 94.361) (end 68.8848 96.6216) (width 3) (layer F.Cu) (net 4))
 (segment (start 71.1454 84.1756) (end 71.1454 94.361) (width 3) (layer F.Cu) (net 4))
 (segment (start 79.0448 100.1644) (end 79.0448 105.8164) (width 3) (layer F.Cu) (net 4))
 (segment (start 79.0448 105.8164) (end 76.6064 108.2548) (width 3) (layer F.Cu) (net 4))
 (segment (start 76.6064 108.2548) (end 72.4916 108.2548) (width 3) (layer F.Cu) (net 4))
 (segment (start 68.8848 104.648) (end 68.8848 96.6216) (width 3) (layer F.Cu) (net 4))
 (segment (start 72.4916 108.2548) (end 68.8848 104.648) (width 3) (layer F.Cu) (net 4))
 (segment (start 94.2858 76.3524) (end 94.362 76.2762) (width 3) (layer F.Cu) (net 4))
 (segment (start 90.551 76.3524) (end 94.2858 76.3524) (width 3) (layer F.Cu) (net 4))
 (segment (start 94.362 76.6074) (end 102.8192 85.0646) (width 2) (layer F.Cu) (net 4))
 (segment (start 94.362 76.2762) (end 94.362 76.6074) (width 2) (layer F.Cu) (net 4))
 (segment (start 101.884 85.0646) (end 98.3742 88.5744) (width 1.5) (layer F.Cu) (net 4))
 (segment (start 102.8192 85.0646) (end 101.884 85.0646) (width 1.5) (layer F.Cu) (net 4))
 (segment (start 78.9178 77.597) (end 78.6892 77.8256) (width 1.5) (layer F.Cu) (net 8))
 (segment (start 78.9178 66.3702) (end 78.9178 77.597) (width 1.5) (layer F.Cu) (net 8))
 (segment (start 78.9178 66.3702) (end 78.9178 66.421) (width 1.5) (layer F.Cu) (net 8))
 (segment (start 81.782 79.635) (end 81.782 73.152) (width 1.5) (layer F.Cu) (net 8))
 (segment (start 77.47 77.8256) (end 76.3524 78.9432) (width 1.5) (layer F.Cu) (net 8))
 (segment (start 76.3524 80.264) (end 76.962 80.8736) (width 1.5) (layer F.Cu) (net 8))
 (segment (start 78.6892 77.8256) (end 77.47 77.8256) (width 1.5) (layer F.Cu) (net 8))
 (segment (start 76.3524 78.9432) (end 76.3524 80.264) (width 1.5) (layer F.Cu) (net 8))
 (segment (start 76.962 80.8736) (end 80.5434 80.8736) (width 1.5) (layer F.Cu) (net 8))
 (segment (start 80.5434 80.8736) (end 81.782 79.635) (width 1.5) (layer F.Cu) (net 8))
 (segment (start 78.6892 77.8256) (end 78.6892 77.2414) (width 3) (layer F.Cu) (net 8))
 (segment (start 76.7334 75.2856) (end 68.9864 75.2856) (width 3) (layer F.Cu) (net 8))
 (segment (start 78.6892 77.2414) (end 76.7334 75.2856) (width 3) (layer F.Cu) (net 8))
 (segment (start 96.2198 60.8076) (end 93.505 60.8076) (width 0.6) (layer F.Cu) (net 3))
 (segment (start 96.8248 60.2026) (end 96.2198 60.8076) (width 0.6) (layer F.Cu) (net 3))
 (segment (start 102.362 76.2762) (end 99.4918 73.406) (width 1.5) (layer F.Cu) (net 3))
 (segment (start 99.4918 73.406) (end 99.4918 60.452) (width 1.5) (layer F.Cu) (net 3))
 (segment (start 99.2424 60.2026) (end 96.8248 60.2026) (width 1.5) (layer F.Cu) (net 3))
 (segment (start 99.4918 60.452) (end 99.2424 60.2026) (width 1.5) (layer F.Cu) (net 3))
 (segment (start 103.632 75.0062) (end 102.362 76.2762) (width 1.5) (layer F.Cu) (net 3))
 (segment (start 103.632 66.6242) (end 103.632 75.0062) (width 1.5) (layer F.Cu) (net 3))
 (segment (start 96.9264 94.2762) (end 98.4082 94.2762) (width 1.5) (layer F.Cu) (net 3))
 (segment (start 98.4082 94.2762) (end 106.172 86.5124) (width 1.5) (layer F.Cu) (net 3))
 (segment (start 106.172 80.0862) (end 102.362 76.2762) (width 1.5) (layer F.Cu) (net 3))
 (segment (start 106.172 86.5124) (end 106.172 80.0862) (width 1.5) (layer F.Cu) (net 3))
 (segment (start 98.3742 94.2422) (end 98.4082 94.2762) (width 1.5) (layer F.Cu) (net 3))
 (segment (start 98.3742 90.4494) (end 98.3742 94.2422) (width 1.5) (layer F.Cu) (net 3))
 (segment (start 90.6028 95.2124) (end 90.9574 95.567) (width 1.5) (layer F.Cu) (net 7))
 (segment (start 90.6028 90.5378) (end 90.6028 95.2124) (width 1.5) (layer F.Cu) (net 7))
 (segment (start 90.7796 95.7448) (end 90.9574 95.567) (width 1.5) (layer F.Cu) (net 7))
 (segment (start 90.7796 100.774) (end 90.7796 95.7448) (width 1.5) (layer F.Cu) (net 7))
 (segment (start 90.7796 100.774) (end 90.7796 111.1626) (width 1.5) (layer F.Cu) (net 7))
 (segment (start 89.8652 112.077) (end 84.7364 112.077) (width 1.5) (layer F.Cu) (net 7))
 (segment (start 90.7796 111.1626) (end 89.8652 112.077) (width 1.5) (layer F.Cu) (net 7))
 (segment (start 91.5924 96.202) (end 90.9574 95.567) (width 0.6) (layer F.Cu) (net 7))
 (segment (start 93.6574 96.202) (end 91.5924 96.202) (width 0.6) (layer F.Cu) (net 7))
 (segment (start 69.5452 118.1608) (end 69.3166 117.9322) (width 3) (layer F.Cu) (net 7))
 (segment (start 82.1436 118.1608) (end 69.5452 118.1608) (width 3) (layer F.Cu) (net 7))
 (segment (start 85.0158 111.8108) (end 85.0158 115.2886) (width 3) (layer F.Cu) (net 7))
 (segment (start 85.0158 115.2886) (end 82.1436 118.1608) (width 3) (layer F.Cu) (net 7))
 (segment (start 93.6244 63.3476) (end 96.2914 66.0146) (width 0.6) (layer F.Cu) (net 9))
 (segment (start 93.505 63.3476) (end 93.6244 63.3476) (width 0.6) (layer F.Cu) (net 9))
 (segment (start 94.1578 97.472) (end 96.647 99.9612) (width 0.6) (layer F.Cu) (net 10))
 (segment (start 93.6574 97.472) (end 94.1578 97.472) (width 0.6) (layer F.Cu) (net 10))
 (segment (start 88.105 63.3476) (end 86.2076 63.3476) (width 0.6) (layer F.Cu) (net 11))
 (segment (start 84.5788 64.9764) (end 84.5788 69.8754) (width 0.6) (layer F.Cu) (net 11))
 (segment (start 86.2076 63.3476) (end 84.5788 64.9764) (width 0.6) (layer F.Cu) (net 11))
 (segment (start 84.5788 73.1488) (end 84.582 73.152) (width 1.5) (layer F.Cu) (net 11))
 (segment (start 84.5788 69.8754) (end 84.5788 73.1488) (width 1.5) (layer F.Cu) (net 11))
 (segment (start 87.576 69.8532) (end 87.5538 69.8754) (width 1.5) (layer F.Cu) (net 17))
 (segment (start 87.576 66.3956) (end 87.576 69.8532) (width 1.5) (layer F.Cu) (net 17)))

